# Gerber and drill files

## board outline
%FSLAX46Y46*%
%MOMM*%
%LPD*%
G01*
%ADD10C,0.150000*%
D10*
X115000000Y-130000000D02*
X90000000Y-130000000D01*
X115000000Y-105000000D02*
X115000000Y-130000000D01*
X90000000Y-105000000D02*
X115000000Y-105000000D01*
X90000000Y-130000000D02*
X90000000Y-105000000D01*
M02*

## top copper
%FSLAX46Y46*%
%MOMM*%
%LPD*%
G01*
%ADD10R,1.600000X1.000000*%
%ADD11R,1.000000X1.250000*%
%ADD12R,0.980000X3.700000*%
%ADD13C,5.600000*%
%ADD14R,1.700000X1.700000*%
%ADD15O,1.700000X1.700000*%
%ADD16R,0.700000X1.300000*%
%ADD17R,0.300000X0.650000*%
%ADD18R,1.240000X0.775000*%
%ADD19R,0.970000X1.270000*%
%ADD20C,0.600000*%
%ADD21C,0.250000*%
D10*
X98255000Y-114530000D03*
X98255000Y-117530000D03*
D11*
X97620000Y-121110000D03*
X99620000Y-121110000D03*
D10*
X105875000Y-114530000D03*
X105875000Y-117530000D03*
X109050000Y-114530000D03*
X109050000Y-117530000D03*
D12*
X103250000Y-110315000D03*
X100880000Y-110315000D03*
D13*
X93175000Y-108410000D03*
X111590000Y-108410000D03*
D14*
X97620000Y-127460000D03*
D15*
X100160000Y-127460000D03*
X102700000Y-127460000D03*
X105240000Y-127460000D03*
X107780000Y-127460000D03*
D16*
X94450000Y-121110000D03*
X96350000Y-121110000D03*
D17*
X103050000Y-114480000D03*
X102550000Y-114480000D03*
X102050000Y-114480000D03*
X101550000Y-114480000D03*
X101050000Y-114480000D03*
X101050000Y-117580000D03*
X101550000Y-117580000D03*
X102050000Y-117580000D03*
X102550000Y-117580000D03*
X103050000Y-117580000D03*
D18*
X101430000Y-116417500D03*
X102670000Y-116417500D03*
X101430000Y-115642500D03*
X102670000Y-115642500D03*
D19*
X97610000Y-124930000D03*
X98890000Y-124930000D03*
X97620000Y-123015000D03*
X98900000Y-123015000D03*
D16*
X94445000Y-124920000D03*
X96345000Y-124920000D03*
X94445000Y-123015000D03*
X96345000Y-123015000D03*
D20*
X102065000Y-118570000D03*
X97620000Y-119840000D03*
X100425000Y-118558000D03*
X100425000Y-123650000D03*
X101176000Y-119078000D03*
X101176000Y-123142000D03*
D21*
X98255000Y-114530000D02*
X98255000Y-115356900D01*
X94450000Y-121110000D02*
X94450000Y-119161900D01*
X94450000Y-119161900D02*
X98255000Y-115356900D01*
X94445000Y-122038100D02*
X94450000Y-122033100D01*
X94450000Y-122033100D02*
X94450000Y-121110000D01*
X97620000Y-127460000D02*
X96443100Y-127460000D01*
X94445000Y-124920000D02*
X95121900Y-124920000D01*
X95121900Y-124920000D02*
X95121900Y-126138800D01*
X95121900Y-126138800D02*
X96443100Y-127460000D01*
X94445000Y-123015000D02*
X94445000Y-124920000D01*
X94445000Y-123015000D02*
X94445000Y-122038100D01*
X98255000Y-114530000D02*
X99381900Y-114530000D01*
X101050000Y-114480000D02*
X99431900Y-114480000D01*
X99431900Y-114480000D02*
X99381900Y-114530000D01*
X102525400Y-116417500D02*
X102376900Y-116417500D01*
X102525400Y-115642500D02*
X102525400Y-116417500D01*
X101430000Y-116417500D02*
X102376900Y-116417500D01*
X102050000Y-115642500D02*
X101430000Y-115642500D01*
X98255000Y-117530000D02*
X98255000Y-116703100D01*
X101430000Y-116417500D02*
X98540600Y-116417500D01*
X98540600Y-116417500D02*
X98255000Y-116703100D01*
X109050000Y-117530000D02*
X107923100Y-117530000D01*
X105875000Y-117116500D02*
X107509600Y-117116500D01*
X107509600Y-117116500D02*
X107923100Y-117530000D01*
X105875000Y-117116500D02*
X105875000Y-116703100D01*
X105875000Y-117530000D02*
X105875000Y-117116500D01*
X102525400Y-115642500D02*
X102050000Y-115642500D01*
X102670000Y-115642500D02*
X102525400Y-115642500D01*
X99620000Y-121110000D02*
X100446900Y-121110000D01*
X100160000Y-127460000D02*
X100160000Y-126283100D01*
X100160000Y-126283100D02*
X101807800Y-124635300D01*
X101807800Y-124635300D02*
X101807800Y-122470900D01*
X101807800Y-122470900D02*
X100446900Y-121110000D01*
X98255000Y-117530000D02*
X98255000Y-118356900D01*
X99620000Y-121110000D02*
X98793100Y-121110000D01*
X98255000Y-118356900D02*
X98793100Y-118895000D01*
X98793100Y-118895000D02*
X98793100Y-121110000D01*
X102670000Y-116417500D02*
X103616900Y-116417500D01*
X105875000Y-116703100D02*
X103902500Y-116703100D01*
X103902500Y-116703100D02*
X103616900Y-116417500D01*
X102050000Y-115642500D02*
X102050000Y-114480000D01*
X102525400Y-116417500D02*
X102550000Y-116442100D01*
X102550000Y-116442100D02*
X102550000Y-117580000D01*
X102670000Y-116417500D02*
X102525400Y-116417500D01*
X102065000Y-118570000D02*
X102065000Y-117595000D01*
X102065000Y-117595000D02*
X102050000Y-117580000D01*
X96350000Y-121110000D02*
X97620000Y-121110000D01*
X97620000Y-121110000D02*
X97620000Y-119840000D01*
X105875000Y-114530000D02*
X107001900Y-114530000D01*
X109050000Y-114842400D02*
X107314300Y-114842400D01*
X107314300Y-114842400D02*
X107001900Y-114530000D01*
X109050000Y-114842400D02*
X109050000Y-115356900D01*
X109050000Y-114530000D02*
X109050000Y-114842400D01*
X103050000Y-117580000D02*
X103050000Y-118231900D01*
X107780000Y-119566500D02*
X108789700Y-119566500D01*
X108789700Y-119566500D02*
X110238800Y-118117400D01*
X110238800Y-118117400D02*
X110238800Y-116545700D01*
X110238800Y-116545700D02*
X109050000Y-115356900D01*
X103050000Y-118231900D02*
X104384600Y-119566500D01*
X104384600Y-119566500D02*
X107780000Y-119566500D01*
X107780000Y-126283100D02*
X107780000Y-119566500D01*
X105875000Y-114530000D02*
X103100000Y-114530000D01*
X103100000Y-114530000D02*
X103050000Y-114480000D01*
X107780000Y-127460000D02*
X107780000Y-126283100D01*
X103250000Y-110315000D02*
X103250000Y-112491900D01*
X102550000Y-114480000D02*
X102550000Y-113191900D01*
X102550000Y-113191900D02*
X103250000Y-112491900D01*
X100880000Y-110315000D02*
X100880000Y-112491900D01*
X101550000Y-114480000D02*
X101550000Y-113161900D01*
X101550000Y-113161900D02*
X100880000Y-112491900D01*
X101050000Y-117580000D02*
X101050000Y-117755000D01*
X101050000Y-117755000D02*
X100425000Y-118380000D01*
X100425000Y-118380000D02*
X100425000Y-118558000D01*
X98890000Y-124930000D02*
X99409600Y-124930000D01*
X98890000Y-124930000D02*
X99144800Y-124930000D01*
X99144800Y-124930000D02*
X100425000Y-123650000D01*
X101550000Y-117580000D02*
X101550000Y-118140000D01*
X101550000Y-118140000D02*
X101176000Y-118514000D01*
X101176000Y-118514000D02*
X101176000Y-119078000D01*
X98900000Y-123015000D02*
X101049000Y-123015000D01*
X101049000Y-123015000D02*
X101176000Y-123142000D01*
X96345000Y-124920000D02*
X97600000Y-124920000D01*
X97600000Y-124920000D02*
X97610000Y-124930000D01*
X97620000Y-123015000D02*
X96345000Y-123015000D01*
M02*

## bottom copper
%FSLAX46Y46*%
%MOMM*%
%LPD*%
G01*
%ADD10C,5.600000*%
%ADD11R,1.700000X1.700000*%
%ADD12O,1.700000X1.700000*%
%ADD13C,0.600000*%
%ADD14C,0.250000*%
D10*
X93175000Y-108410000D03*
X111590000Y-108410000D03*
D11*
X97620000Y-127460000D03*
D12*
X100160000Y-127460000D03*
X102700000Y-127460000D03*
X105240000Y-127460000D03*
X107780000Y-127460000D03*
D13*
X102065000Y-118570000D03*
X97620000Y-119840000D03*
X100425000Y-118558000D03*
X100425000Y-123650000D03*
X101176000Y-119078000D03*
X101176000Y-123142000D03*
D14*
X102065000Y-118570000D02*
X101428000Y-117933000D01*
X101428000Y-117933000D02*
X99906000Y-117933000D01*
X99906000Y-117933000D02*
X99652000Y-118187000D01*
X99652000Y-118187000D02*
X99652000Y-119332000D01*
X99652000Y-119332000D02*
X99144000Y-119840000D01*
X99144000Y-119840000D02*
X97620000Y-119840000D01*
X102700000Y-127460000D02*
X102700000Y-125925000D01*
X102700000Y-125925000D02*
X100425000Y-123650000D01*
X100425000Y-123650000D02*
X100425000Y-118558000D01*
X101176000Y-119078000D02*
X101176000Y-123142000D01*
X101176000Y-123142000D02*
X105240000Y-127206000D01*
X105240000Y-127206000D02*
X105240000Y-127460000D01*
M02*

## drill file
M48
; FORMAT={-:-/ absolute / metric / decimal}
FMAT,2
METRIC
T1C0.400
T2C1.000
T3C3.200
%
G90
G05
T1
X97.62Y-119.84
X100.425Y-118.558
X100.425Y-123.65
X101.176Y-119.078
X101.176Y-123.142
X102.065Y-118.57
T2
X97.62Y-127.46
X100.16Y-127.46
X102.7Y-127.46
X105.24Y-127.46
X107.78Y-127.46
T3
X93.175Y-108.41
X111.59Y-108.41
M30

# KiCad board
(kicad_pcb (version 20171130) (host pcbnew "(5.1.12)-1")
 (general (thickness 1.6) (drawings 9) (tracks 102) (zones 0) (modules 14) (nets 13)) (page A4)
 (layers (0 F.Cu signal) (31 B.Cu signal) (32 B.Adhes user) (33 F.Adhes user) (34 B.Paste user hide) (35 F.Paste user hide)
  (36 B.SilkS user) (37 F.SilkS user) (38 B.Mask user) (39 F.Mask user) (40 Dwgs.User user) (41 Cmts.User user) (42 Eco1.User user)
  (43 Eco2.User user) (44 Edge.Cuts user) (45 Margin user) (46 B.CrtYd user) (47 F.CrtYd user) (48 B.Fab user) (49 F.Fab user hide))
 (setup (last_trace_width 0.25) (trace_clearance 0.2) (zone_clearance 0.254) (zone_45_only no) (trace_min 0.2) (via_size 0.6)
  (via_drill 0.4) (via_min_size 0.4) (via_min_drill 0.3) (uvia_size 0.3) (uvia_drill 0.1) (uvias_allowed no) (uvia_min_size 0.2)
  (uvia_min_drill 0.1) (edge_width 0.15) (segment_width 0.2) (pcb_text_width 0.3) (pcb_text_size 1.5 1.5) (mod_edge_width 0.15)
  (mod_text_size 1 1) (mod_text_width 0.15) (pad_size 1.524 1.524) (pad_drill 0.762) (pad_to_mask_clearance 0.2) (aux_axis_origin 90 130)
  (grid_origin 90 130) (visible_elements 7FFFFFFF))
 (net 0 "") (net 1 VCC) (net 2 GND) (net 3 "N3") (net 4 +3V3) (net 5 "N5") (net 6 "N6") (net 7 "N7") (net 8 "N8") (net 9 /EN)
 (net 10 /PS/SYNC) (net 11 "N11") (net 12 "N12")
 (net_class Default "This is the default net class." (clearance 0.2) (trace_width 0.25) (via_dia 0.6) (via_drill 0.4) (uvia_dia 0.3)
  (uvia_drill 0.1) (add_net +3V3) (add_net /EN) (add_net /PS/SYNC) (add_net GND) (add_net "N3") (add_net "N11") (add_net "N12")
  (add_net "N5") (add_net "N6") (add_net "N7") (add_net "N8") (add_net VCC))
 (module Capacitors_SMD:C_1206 (layer F.Cu) (at 98.255 116.03 270)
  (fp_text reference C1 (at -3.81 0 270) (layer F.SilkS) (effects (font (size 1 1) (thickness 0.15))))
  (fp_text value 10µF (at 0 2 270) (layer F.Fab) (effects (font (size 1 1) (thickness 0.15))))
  (pad 1 smd rect (at -1.5 0 270) (size 1 1.6) (layers F.Cu F.Paste F.Mask) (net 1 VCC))
  (pad 2 smd rect (at 1.5 0 270) (size 1 1.6) (layers F.Cu F.Paste F.Mask) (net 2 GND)))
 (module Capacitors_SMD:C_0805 (layer F.Cu) (at 98.62 121.11)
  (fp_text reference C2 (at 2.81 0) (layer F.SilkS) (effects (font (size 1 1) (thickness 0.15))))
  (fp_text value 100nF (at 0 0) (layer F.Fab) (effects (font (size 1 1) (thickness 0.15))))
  (pad 1 smd rect (at -1 0) (size 1 1.25) (layers F.Cu F.Paste F.Mask) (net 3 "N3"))
  (pad 2 smd rect (at 1 0) (size 1 1.25) (layers F.Cu F.Paste F.Mask) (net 2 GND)))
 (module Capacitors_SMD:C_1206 (layer F.Cu) (at 105.875 116.03 270)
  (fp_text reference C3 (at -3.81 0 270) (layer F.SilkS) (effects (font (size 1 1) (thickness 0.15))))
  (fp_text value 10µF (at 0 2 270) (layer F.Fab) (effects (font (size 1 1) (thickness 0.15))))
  (pad 1 smd rect (at -1.5 0 270) (size 1 1.6) (layers F.Cu F.Paste F.Mask) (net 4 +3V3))
  (pad 2 smd rect (at 1.5 0 270) (size 1 1.6) (layers F.Cu F.Paste F.Mask) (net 2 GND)))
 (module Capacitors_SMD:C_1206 (layer F.Cu) (at 109.05 116.03 270)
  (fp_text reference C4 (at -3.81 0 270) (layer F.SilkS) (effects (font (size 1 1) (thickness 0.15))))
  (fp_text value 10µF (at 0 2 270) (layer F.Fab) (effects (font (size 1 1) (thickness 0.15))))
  (pad 1 smd rect (at -1.5 0 270) (size 1 1.6) (layers F.Cu F.Paste F.Mask) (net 4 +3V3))
  (pad 2 smd rect (at 1.5 0 270) (size 1 1.6) (layers F.Cu F.Paste F.Mask) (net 2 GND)))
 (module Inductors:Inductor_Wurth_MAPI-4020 (layer F.Cu) (at 102.065 110.315 180)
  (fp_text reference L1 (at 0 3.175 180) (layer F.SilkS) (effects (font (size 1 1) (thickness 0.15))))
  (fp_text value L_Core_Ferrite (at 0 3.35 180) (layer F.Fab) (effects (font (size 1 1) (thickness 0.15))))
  (pad 1 smd rect (at -1.185 0 180) (size 0.98 3.7) (layers F.Cu F.Paste F.Mask) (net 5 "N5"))
  (pad 2 smd rect (at 1.185 0 180) (size 0.98 3.7) (layers F.Cu F.Paste F.Mask) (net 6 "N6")))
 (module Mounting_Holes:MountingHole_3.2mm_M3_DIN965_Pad (layer F.Cu) (at 93.175 108.41)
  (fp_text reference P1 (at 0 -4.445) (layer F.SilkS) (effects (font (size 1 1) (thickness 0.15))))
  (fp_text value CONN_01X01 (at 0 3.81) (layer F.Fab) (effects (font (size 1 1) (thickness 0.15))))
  (pad 1 thru_hole circle (at 0 0) (size 5.6 5.6) (drill 3.2) (layers *.Cu *.Mask) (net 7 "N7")))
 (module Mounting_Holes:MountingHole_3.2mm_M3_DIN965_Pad (layer F.Cu) (at 111.59 108.41)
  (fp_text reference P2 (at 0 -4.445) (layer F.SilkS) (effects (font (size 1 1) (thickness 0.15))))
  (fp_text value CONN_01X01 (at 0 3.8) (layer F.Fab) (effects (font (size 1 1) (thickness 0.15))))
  (pad 1 thru_hole circle (at 0 0) (size 5.6 5.6) (drill 3.2) (layers *.Cu *.Mask) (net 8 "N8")))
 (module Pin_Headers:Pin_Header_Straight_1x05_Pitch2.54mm (layer F.Cu) (at 97.62 127.46 90)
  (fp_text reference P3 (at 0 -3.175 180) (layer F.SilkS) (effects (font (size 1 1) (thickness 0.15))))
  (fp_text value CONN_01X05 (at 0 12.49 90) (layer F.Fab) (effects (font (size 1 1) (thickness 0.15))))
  (pad 1 thru_hole rect (at 0 0 90) (size 1.7 1.7) (drill 1) (layers *.Cu *.Mask) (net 1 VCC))
  (pad 2 thru_hole oval (at 0 2.54 90) (size 1.7 1.7) (drill 1) (layers *.Cu *.Mask) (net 2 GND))
  (pad 3 thru_hole oval (at 0 5.08 90) (size 1.7 1.7) (drill 1) (layers *.Cu *.Mask) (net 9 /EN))
  (pad 4 thru_hole oval (at 0 7.62 90) (size 1.7 1.7) (drill 1) (layers *.Cu *.Mask) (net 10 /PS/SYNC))
  (pad 5 thru_hole oval (at 0 10.16 90) (size 1.7 1.7) (drill 1) (layers *.Cu *.Mask) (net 4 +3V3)))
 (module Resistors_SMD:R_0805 (layer F.Cu) (at 95.4 121.11)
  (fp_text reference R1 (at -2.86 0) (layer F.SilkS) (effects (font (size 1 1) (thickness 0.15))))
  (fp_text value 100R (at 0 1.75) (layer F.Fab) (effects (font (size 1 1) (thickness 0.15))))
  (pad 1 smd rect (at -0.95 0) (size 0.7 1.3) (layers F.Cu F.Paste F.Mask) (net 1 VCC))
  (pad 2 smd rect (at 0.95 0) (size 0.7 1.3) (layers F.Cu F.Paste F.Mask) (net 3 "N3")))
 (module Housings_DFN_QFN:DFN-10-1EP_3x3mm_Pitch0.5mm (layer F.Cu) (at 102.05 116.03 270)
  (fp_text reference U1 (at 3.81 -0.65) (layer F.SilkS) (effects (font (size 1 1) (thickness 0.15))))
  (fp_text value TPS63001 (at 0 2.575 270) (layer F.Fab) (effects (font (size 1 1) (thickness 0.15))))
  (pad 1 smd rect (at -1.55 -1 270) (size 0.65 0.3) (layers F.Cu F.Paste F.Mask) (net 4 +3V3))
  (pad 2 smd rect (at -1.55 -0.5 270) (size 0.65 0.3) (layers F.Cu F.Paste F.Mask) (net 5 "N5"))
  (pad 3 smd rect (at -1.55 0 270) (size 0.65 0.3) (layers F.Cu F.Paste F.Mask) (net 2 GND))
  (pad 4 smd rect (at -1.55 0.5 270) (size 0.65 0.3) (layers F.Cu F.Paste F.Mask) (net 6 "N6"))
  (pad 5 smd rect (at -1.55 1 270) (size 0.65 0.3) (layers F.Cu F.Paste F.Mask) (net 1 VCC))
  (pad 6 smd rect (at 1.55 1 270) (size 0.65 0.3) (layers F.Cu F.Paste F.Mask) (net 9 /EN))
  (pad 7 smd rect (at 1.55 0.5 270) (size 0.65 0.3) (layers F.Cu F.Paste F.Mask) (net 10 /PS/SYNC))
  (pad 8 smd rect (at 1.55 0 270) (size 0.65 0.3) (layers F.Cu F.Paste F.Mask) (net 3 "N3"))
  (pad 9 smd rect (at 1.55 -0.5 270) (size 0.65 0.3) (layers F.Cu F.Paste F.Mask) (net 2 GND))
  (pad 10 smd rect (at 1.55 -1 270) (size 0.65 0.3) (layers F.Cu F.Paste F.Mask) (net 4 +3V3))
  (pad 11 smd rect (at 0.3875 0.62 270) (size 0.775 1.24) (layers F.Cu F.Paste F.Mask) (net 2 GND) (solder_paste_margin_ratio -0.2))
  (pad 11 smd rect (at 0.3875 -0.62 270) (size 0.775 1.24) (layers F.Cu F.Paste F.Mask) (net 2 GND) (solder_paste_margin_ratio -0.2))
  (pad 11 smd rect (at -0.3875 0.62 270) (size 0.775 1.24) (layers F.Cu F.Paste F.Mask) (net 2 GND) (solder_paste_margin_ratio -0.2))
  (pad 11 smd rect (at -0.3875 -0.62 270) (size 0.775 1.24) (layers F.Cu F.Paste F.Mask) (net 2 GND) (solder_paste_margin_ratio -0.2)))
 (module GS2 (layer F.Cu) (at 98.25 124.93 90)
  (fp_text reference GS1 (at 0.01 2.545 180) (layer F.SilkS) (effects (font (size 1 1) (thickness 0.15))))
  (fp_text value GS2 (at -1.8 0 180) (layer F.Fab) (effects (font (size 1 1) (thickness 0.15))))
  (pad 1 smd rect (at 0 -0.64 90) (size 1.27 0.97) (layers F.Cu F.Paste F.Mask) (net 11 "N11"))
  (pad 2 smd rect (at 0 0.64 90) (size 1.27 0.97) (layers F.Cu F.Paste F.Mask) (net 9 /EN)))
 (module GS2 (layer F.Cu) (at 98.26 123.015 90)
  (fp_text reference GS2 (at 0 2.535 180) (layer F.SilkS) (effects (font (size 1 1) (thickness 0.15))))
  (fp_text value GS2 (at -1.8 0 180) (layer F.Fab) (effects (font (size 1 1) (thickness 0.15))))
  (pad 1 smd rect (at 0 -0.64 90) (size 1.27 0.97) (layers F.Cu F.Paste F.Mask) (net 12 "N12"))
  (pad 2 smd rect (at 0 0.64 90) (size 1.27 0.97) (layers F.Cu F.Paste F.Mask) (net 10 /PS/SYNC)))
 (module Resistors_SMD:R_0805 (layer F.Cu) (at 95.395 124.92)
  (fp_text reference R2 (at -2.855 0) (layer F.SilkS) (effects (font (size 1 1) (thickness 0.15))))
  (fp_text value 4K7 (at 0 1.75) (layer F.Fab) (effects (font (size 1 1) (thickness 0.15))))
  (pad 1 smd rect (at -0.95 0) (size 0.7 1.3) (layers F.Cu F.Paste F.Mask) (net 1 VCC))
  (pad 2 smd rect (at 0.95 0) (size 0.7 1.3) (layers F.Cu F.Paste F.Mask) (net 11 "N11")))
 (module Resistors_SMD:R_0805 (layer F.Cu) (at 95.395 123.015)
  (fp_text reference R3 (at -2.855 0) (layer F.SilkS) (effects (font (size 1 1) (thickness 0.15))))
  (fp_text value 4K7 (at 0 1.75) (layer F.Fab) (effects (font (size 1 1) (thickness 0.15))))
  (pad 1 smd rect (at -0.95 0) (size 0.7 1.3) (layers F.Cu F.Paste F.Mask) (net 1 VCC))
  (pad 2 smd rect (at 0.95 0) (size 0.7 1.3) (layers F.Cu F.Paste F.Mask) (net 12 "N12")))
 (gr_line (start 115 130) (end 90 130) (layer Edge.Cuts) (width 0.15))
 (gr_line (start 115 105) (end 115 130) (layer Edge.Cuts) (width 0.15))
 (gr_line (start 90 105) (end 115 105) (layer Edge.Cuts) (width 0.15))
 (gr_line (start 90 130) (end 90 105) (layer Edge.Cuts) (width 0.15))
 (segment (start 98.255 114.53) (end 98.255 115.3569) (width 0.25) (layer F.Cu) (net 1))
 (segment (start 94.45 121.11) (end 94.45 119.1619) (width 0.25) (layer F.Cu) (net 1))
 (segment (start 94.45 119.1619) (end 98.255 115.3569) (width 0.25) (layer F.Cu) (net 1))
 (segment (start 94.445 122.0381) (end 94.45 122.0331) (width 0.25) (layer F.Cu) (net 1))
 (segment (start 94.45 122.0331) (end 94.45 121.11) (width 0.25) (layer F.Cu) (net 1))
 (segment (start 97.62 127.46) (end 96.4431 127.46) (width 0.25) (layer F.Cu) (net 1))
 (segment (start 94.445 124.92) (end 95.1219 124.92) (width 0.25) (layer F.Cu) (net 1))
 (segment (start 95.1219 124.92) (end 95.1219 126.1388) (width 0.25) (layer F.Cu) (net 1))
 (segment (start 95.1219 126.1388) (end 96.4431 127.46) (width 0.25) (layer F.Cu) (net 1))
 (segment (start 94.445 123.015) (end 94.445 124.92) (width 0.25) (layer F.Cu) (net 1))
 (segment (start 94.445 123.015) (end 94.445 122.0381) (width 0.25) (layer F.Cu) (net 1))
 (segment (start 98.255 114.53) (end 99.3819 114.53) (width 0.25) (layer F.Cu) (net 1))
 (segment (start 101.05 114.48) (end 99.4319 114.48) (width 0.25) (layer F.Cu) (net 1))
 (segment (start 99.4319 114.48) (end 99.3819 114.53) (width 0.25) (layer F.Cu) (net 1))
 (segment (start 102.5254 116.4175) (end 102.3769 116.4175) (width 0.25) (layer F.Cu) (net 2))
 (segment (start 102.5254 115.6425) (end 102.5254 116.4175) (width 0.25) (layer F.Cu) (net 2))
 (segment (start 101.43 116.4175) (end 102.3769 116.4175) (width 0.25) (layer F.Cu) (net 2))
 (segment (start 102.05 115.6425) (end 101.43 115.6425) (width 0.25) (layer F.Cu) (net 2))
 (segment (start 98.255 117.53) (end 98.255 116.7031) (width 0.25) (layer F.Cu) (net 2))
 (segment (start 101.43 116.4175) (end 98.5406 116.4175) (width 0.25) (layer F.Cu) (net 2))
 (segment (start 98.5406 116.4175) (end 98.255 116.7031) (width 0.25) (layer F.Cu) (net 2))
 (segment (start 109.05 117.53) (end 107.9231 117.53) (width 0.25) (layer F.Cu) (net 2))
 (segment (start 105.875 117.1165) (end 107.5096 117.1165) (width 0.25) (layer F.Cu) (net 2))
 (segment (start 107.5096 117.1165) (end 107.9231 117.53) (width 0.25) (layer F.Cu) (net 2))
 (segment (start 105.875 117.1165) (end 105.875 116.7031) (width 0.25) (layer F.Cu) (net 2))
 (segment (start 105.875 117.53) (end 105.875 117.1165) (width 0.25) (layer F.Cu) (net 2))
 (segment (start 102.5254 115.6425) (end 102.05 115.6425) (width 0.25) (layer F.Cu) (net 2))
 (segment (start 102.67 115.6425) (end 102.5254 115.6425) (width 0.25) (layer F.Cu) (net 2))
 (segment (start 99.62 121.11) (end 100.4469 121.11) (width 0.25) (layer F.Cu) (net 2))
 (segment (start 100.16 127.46) (end 100.16 126.2831) (width 0.25) (layer F.Cu) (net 2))
 (segment (start 100.16 126.2831) (end 101.8078 124.6353) (width 0.25) (layer F.Cu) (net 2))
 (segment (start 101.8078 124.6353) (end 101.8078 122.4709) (width 0.25) (layer F.Cu) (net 2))
 (segment (start 101.8078 122.4709) (end 100.4469 121.11) (width 0.25) (layer F.Cu) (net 2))
 (segment (start 98.255 117.53) (end 98.255 118.3569) (width 0.25) (layer F.Cu) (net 2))
 (segment (start 99.62 121.11) (end 98.7931 121.11) (width 0.25) (layer F.Cu) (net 2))
 (segment (start 98.255 118.3569) (end 98.7931 118.895) (width 0.25) (layer F.Cu) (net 2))
 (segment (start 98.7931 118.895) (end 98.7931 121.11) (width 0.25) (layer F.Cu) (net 2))
 (segment (start 102.67 116.4175) (end 103.6169 116.4175) (width 0.25) (layer F.Cu) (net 2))
 (segment (start 105.875 116.7031) (end 103.9025 116.7031) (width 0.25) (layer F.Cu) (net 2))
 (segment (start 103.9025 116.7031) (end 103.6169 116.4175) (width 0.25) (layer F.Cu) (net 2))
 (segment (start 102.05 115.6425) (end 102.05 114.48) (width 0.25) (layer F.Cu) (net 2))
 (segment (start 102.5254 116.4175) (end 102.55 116.4421) (width 0.25) (layer F.Cu) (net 2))
 (segment (start 102.55 116.4421) (end 102.55 117.58) (width 0.25) (layer F.Cu) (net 2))
 (segment (start 102.67 116.4175) (end 102.5254 116.4175) (width 0.25) (layer F.Cu) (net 2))
 (segment (start 102.065 118.57) (end 102.065 117.595) (width 0.25) (layer F.Cu) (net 3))
 (segment (start 102.065 117.595) (end 102.05 117.58) (width 0.25) (layer F.Cu) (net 3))
 (segment (start 96.35 121.11) (end 97.62 121.11) (width 0.25) (layer F.Cu) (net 3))
 (segment (start 97.62 121.11) (end 97.62 119.84) (width 0.25) (layer F.Cu) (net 3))
 (segment (start 102.065 118.57) (end 101.428 117.933) (width 0.25) (layer B.Cu) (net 3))
 (segment (start 101.428 117.933) (end 99.906 117.933) (width 0.25) (layer B.Cu) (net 3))
 (segment (start 99.906 117.933) (end 99.652 118.187) (width 0.25) (layer B.Cu) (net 3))
 (segment (start 99.652 118.187) (end 99.652 119.332) (width 0.25) (layer B.Cu) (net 3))
 (segment (start 99.652 119.332) (end 99.144 119.84) (width 0.25) (layer B.Cu) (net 3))
 (segment (start 99.144 119.84) (end 97.62 119.84) (width 0.25) (layer B.Cu) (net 3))
 (via (at 102.065 118.57) (size 0.6) (layers F.Cu B.Cu) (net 3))
 (via (at 97.62 119.84) (size 0.6) (layers F.Cu B.Cu) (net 3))
 (segment (start 105.875 114.53) (end 107.0019 114.53) (width 0.25) (layer F.Cu) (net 4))
 (segment (start 109.05 114.8424) (end 107.3143 114.8424) (width 0.25) (layer F.Cu) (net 4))
 (segment (start 107.3143 114.8424) (end 107.0019 114.53) (width 0.25) (layer F.Cu) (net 4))
 (segment (start 109.05 114.8424) (end 109.05 115.3569) (width 0.25) (layer F.Cu) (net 4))
 (segment (start 109.05 114.53) (end 109.05 114.8424) (width 0.25) (layer F.Cu) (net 4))
 (segment (start 103.05 117.58) (end 103.05 118.2319) (width 0.25) (layer F.Cu) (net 4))
 (segment (start 107.78 119.5665) (end 108.7897 119.5665) (width 0.25) (layer F.Cu) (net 4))
 (segment (start 108.7897 119.5665) (end 110.2388 118.1174) (width 0.25) (layer F.Cu) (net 4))
 (segment (start 110.2388 118.1174) (end 110.2388 116.5457) (width 0.25) (layer F.Cu) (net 4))
 (segment (start 110.2388 116.5457) (end 109.05 115.3569) (width 0.25) (layer F.Cu) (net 4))
 (segment (start 103.05 118.2319) (end 104.3846 119.5665) (width 0.25) (layer F.Cu) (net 4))
 (segment (start 104.3846 119.5665) (end 107.78 119.5665) (width 0.25) (layer F.Cu) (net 4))
 (segment (start 107.78 126.2831) (end 107.78 119.5665) (width 0.25) (layer F.Cu) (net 4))
 (segment (start 105.875 114.53) (end 103.1 114.53) (width 0.25) (layer F.Cu) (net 4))
 (segment (start 103.1 114.53) (end 103.05 114.48) (width 0.25) (layer F.Cu) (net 4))
 (segment (start 107.78 127.46) (end 107.78 126.2831) (width 0.25) (layer F.Cu) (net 4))
 (segment (start 103.25 110.315) (end 103.25 112.4919) (width 0.25) (layer F.Cu) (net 5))
 (segment (start 102.55 114.48) (end 102.55 113.1919) (width 0.25) (layer F.Cu) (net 5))
 (segment (start 102.55 113.1919) (end 103.25 112.4919) (width 0.25) (layer F.Cu) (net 5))
 (segment (start 100.88 110.315) (end 100.88 112.4919) (width 0.25) (layer F.Cu) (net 6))
 (segment (start 101.55 114.48) (end 101.55 113.1619) (width 0.25) (layer F.Cu) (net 6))
 (segment (start 101.55 113.1619) (end 100.88 112.4919) (width 0.25) (layer F.Cu) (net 6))
 (segment (start 101.05 117.58) (end 101.05 117.755) (width 0.25) (layer F.Cu) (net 9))
 (segment (start 101.05 117.755) (end 100.425 118.38) (width 0.25) (layer F.Cu) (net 9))
 (segment (start 100.425 118.38) (end 100.425 118.558) (width 0.25) (layer F.Cu) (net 9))
 (segment (start 102.7 127.46) (end 102.7 125.925) (width 0.25) (layer B.Cu) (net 9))
 (segment (start 102.7 125.925) (end 100.425 123.65) (width 0.25) (layer B.Cu) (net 9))
 (segment (start 98.89 124.93) (end 99.4096 124.93) (width 0.25) (layer F.Cu) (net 9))
 (segment (start 100.425 123.65) (end 100.425 118.558) (width 0.25) (layer B.Cu) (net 9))
 (segment (start 98.89 124.93) (end 99.1448 124.93) (width 0.25) (layer F.Cu) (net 9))
 (segment (start 99.1448 124.93) (end 100.425 123.65) (width 0.25) (layer F.Cu) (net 9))
 (via (at 100.425 118.558) (size 0.6) (layers F.Cu B.Cu) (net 9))
 (via (at 100.425 123.65) (size 0.6) (layers F.Cu B.Cu) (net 9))
 (segment (start 101.55 117.58) (end 101.55 118.14) (width 0.25) (layer F.Cu) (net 10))
 (segment (start 101.55 118.14) (end 101.176 118.514) (width 0.25) (layer F.Cu) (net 10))
 (segment (start 101.176 118.514) (end 101.176 119.078) (width 0.25) (layer F.Cu) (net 10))
 (segment (start 98.9 123.015) (end 101.049 123.015) (width 0.25) (layer F.Cu) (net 10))
 (segment (start 101.049 123.015) (end 101.176 123.142) (width 0.25) (layer F.Cu) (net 10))
 (segment (start 101.176 119.078) (end 101.176 123.142) (width 0.25) (layer B.Cu) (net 10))
 (segment (start 101.176 123.142) (end 105.24 127.206) (width 0.25) (layer B.Cu) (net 10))
 (segment (start 105.24 127.206) (end 105.24 127.46) (width 0.25) (layer B.Cu) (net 10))
 (via (at 101.176 119.078) (size 0.6) (layers F.Cu B.Cu) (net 10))
 (via (at 101.176 123.142) (size 0.6) (layers F.Cu B.Cu) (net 10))
 (segment (start 96.345 124.92) (end 97.6 124.92) (width 0.25) (layer F.Cu) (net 11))
 (segment (start 97.6 124.92) (end 97.61 124.93) (width 0.25) (layer F.Cu) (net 11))
 (segment (start 97.62 123.015) (end 96.345 123.015) (width 0.25) (layer F.Cu) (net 12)))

